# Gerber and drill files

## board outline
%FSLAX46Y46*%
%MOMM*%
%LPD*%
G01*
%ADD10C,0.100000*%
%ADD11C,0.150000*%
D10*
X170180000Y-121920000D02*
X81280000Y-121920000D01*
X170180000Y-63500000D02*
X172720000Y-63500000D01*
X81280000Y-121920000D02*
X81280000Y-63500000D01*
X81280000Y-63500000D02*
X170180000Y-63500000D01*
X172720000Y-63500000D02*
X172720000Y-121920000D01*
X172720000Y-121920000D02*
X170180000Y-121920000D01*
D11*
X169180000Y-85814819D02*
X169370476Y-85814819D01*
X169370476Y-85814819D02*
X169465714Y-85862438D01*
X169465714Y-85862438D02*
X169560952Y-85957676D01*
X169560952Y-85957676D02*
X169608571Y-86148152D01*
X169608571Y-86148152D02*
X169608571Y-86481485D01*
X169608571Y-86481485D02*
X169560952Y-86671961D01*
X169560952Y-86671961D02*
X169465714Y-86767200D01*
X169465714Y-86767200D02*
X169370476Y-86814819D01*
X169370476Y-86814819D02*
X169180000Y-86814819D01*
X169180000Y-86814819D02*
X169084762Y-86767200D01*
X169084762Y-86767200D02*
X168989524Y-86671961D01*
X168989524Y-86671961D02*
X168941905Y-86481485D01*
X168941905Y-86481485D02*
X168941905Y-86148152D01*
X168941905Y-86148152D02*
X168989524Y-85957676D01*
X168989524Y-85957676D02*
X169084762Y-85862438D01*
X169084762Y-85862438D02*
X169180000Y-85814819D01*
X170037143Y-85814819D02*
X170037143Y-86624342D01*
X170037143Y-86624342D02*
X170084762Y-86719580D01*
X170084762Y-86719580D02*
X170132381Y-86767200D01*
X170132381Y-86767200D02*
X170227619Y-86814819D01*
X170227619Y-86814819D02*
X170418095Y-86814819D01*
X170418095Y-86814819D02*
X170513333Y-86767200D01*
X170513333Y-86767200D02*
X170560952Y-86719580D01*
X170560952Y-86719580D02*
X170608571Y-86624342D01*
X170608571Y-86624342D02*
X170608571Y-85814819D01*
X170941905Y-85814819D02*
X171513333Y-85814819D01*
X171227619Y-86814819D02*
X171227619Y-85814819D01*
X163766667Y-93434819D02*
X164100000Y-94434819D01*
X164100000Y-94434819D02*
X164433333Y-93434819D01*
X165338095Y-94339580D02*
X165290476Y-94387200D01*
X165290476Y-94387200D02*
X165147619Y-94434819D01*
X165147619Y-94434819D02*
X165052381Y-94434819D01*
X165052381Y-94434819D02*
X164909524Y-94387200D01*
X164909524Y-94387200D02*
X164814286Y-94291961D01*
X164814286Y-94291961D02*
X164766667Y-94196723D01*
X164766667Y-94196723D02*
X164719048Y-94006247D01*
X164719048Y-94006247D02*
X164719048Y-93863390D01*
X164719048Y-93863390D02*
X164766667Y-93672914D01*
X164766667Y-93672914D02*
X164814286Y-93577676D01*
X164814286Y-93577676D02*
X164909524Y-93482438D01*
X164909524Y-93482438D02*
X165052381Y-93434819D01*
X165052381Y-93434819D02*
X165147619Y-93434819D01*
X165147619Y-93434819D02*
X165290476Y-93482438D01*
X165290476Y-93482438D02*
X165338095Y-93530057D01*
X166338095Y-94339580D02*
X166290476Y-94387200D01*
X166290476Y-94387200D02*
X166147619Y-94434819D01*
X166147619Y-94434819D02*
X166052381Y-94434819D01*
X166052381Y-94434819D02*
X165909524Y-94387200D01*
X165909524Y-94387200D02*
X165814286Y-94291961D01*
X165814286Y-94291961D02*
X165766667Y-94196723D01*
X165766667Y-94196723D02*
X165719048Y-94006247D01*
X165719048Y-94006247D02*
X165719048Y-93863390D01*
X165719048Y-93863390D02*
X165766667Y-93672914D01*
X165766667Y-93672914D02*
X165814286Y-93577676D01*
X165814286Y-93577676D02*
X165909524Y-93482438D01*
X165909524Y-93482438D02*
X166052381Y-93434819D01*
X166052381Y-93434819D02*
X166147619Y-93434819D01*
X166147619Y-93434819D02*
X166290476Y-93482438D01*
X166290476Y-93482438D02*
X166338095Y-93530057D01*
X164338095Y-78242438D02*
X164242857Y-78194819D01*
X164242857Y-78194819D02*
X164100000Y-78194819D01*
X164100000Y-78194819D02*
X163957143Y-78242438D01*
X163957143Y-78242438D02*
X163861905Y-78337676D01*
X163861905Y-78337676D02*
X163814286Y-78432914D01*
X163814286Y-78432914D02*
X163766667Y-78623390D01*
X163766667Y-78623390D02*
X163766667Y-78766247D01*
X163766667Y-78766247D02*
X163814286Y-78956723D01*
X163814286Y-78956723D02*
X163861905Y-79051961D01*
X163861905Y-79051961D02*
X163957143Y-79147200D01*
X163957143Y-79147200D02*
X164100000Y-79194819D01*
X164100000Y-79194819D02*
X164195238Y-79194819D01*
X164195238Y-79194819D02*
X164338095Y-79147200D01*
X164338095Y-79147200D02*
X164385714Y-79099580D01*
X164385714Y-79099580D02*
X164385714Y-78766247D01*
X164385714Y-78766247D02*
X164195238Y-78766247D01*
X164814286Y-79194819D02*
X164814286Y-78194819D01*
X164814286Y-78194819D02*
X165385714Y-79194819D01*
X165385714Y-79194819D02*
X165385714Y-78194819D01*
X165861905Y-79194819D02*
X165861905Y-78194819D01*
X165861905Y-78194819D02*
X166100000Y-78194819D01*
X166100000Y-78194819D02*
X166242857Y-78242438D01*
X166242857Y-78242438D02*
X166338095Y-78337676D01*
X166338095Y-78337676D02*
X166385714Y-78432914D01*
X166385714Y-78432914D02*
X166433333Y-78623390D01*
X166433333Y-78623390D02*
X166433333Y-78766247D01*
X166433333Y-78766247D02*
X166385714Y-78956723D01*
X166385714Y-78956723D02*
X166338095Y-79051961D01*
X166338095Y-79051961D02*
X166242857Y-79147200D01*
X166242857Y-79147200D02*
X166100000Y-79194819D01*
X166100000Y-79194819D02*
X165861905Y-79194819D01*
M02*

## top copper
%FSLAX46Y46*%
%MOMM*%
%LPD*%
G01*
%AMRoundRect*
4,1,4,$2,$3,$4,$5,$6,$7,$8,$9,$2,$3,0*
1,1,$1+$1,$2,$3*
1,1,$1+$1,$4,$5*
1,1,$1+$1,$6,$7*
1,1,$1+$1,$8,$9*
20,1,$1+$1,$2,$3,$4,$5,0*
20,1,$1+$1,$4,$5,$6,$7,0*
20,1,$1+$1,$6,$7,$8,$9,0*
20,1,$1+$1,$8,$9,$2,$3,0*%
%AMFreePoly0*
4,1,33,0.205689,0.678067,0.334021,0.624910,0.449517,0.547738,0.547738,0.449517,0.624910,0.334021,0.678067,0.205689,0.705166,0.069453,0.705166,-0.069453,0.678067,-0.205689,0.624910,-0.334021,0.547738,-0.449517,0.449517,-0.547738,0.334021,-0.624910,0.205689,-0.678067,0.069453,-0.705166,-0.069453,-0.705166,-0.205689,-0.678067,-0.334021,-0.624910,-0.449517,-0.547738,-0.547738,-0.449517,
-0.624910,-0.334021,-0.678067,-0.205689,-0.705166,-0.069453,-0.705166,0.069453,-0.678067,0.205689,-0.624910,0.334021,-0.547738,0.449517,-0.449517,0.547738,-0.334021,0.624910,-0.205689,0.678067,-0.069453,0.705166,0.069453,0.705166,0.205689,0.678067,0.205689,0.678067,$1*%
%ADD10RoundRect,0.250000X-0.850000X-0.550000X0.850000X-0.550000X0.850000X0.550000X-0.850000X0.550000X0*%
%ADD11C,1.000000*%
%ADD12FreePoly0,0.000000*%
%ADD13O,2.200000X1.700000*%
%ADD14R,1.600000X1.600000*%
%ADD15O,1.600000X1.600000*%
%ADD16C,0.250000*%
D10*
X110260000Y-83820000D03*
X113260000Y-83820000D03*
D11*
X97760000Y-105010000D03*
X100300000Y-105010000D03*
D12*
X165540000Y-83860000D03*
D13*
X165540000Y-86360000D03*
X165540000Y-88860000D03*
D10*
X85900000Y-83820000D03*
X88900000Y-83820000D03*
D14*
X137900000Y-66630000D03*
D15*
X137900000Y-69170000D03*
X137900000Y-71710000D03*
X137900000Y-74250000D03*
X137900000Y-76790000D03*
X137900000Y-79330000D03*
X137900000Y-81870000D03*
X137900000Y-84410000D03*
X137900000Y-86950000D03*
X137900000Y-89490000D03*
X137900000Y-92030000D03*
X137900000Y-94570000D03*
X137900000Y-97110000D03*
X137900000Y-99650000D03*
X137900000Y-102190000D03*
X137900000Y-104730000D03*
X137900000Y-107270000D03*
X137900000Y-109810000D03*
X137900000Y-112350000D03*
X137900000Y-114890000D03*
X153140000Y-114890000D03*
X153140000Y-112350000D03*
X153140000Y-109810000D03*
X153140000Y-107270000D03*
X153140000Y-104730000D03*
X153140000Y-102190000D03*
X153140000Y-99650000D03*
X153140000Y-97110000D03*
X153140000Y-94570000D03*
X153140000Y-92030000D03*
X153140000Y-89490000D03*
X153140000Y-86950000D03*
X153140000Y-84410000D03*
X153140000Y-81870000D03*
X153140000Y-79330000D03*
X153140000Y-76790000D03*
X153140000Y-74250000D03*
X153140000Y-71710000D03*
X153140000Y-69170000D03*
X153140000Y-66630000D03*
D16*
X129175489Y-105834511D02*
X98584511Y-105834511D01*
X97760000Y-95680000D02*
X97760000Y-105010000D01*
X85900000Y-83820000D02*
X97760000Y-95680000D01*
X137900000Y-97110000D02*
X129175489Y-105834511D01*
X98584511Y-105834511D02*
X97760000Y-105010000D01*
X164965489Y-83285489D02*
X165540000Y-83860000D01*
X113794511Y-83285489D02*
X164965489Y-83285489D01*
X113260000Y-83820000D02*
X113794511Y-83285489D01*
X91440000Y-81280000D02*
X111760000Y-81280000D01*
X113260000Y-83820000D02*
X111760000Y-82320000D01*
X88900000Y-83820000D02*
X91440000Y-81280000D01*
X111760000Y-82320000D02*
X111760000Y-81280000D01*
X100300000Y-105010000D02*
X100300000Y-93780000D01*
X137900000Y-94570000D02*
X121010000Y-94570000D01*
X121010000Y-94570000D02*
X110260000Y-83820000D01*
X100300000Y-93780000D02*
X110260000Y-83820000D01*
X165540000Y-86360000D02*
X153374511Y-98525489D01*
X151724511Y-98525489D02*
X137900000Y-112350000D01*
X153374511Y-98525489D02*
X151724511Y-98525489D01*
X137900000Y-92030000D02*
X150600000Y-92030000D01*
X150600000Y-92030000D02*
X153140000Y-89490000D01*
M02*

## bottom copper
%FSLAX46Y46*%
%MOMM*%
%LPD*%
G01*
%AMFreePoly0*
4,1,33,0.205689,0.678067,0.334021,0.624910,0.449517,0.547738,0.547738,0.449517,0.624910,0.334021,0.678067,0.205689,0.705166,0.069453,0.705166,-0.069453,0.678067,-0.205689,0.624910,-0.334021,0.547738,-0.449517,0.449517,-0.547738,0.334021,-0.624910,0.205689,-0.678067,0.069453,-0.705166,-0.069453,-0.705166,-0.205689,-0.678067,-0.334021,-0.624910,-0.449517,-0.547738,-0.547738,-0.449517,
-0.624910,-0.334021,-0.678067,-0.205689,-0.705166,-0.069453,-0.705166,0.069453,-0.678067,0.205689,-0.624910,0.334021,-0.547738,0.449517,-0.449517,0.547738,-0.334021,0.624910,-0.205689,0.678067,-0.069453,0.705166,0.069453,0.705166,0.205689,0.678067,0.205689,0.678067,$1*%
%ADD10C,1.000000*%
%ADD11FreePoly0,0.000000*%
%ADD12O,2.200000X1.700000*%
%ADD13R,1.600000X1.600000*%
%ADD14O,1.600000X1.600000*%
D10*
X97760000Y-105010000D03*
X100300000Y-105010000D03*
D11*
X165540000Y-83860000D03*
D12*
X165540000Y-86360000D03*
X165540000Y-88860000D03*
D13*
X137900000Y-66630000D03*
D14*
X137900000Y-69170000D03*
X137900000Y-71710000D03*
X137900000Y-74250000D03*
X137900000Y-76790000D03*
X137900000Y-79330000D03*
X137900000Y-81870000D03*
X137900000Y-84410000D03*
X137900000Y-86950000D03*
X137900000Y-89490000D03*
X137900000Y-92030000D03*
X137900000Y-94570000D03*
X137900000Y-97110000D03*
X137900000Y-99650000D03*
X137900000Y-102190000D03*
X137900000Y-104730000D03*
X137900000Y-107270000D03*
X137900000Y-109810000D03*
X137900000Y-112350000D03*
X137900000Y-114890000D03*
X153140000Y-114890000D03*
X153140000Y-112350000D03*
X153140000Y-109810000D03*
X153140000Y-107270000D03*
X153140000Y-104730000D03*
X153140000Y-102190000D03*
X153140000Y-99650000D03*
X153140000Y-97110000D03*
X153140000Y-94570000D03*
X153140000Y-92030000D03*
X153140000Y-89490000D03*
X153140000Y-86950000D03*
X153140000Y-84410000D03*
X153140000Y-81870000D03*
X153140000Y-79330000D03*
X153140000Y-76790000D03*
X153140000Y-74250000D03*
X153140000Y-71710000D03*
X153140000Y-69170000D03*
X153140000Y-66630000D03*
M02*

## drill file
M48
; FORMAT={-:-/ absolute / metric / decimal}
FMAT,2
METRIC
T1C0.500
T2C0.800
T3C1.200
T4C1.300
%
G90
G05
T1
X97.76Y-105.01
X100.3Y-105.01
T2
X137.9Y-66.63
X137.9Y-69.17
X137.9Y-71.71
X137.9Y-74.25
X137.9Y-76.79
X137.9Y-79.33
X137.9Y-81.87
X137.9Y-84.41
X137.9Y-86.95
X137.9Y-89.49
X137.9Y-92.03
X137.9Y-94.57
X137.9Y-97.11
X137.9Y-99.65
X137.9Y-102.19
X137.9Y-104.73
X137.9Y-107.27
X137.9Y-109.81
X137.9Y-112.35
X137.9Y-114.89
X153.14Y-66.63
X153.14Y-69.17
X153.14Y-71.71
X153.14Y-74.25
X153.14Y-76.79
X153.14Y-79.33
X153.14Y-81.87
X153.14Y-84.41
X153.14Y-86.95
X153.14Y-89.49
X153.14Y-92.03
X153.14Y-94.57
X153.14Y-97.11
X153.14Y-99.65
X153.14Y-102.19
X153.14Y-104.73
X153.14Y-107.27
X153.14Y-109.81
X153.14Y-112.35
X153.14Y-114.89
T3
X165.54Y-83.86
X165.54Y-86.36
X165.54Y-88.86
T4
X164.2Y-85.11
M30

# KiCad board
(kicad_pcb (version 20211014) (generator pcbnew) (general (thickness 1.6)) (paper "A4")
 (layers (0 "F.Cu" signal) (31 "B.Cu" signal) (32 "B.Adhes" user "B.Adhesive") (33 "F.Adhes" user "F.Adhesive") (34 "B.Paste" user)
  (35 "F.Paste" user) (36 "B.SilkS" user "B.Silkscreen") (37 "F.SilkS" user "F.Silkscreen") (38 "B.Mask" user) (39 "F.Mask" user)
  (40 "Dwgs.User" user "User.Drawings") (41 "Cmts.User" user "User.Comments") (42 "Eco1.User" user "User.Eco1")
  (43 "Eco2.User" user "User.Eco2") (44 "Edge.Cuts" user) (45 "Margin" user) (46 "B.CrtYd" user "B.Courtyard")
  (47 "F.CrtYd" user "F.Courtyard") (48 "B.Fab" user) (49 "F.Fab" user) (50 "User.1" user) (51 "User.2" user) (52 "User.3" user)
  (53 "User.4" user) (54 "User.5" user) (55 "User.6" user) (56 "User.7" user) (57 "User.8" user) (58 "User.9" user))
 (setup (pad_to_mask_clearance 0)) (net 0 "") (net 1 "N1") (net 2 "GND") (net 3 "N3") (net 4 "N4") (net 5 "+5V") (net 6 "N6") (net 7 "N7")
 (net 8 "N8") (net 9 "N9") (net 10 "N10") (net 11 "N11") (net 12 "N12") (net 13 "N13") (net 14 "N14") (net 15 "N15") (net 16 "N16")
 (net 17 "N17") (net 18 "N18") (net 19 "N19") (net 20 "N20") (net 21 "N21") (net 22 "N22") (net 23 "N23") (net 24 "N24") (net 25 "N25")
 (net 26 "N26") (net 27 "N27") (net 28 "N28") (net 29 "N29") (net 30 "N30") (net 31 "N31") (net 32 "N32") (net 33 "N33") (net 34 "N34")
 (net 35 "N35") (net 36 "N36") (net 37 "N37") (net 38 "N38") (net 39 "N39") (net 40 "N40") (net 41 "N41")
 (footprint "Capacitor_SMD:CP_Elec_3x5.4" (layer "F.Cu") (at 111.76 83.82)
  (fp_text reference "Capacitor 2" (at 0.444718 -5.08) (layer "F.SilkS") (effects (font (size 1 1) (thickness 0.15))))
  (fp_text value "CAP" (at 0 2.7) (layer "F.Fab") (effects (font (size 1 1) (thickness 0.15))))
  (pad "1" smd roundrect (at -1.5 0) (size 2.2 1.6) (layers "F.Cu" "F.Paste" "F.Mask") (roundrect_rratio 0.15625) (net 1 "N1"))
  (pad "2" smd roundrect (at 1.5 0) (size 2.2 1.6) (layers "F.Cu" "F.Paste" "F.Mask") (roundrect_rratio 0.15625) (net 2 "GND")))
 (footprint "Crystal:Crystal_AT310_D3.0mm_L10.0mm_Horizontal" (layer "F.Cu") (at 97.76 105.01)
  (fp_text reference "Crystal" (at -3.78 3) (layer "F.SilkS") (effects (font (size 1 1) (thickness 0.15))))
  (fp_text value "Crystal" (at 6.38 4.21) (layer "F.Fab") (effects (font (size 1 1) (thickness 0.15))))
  (pad "1" thru_hole circle (at 0 0) (size 1 1) (drill 0.5) (layers *.Cu *.Mask) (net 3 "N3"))
  (pad "2" thru_hole circle (at 2.54 0) (size 1 1) (drill 0.5) (layers *.Cu *.Mask) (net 1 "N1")))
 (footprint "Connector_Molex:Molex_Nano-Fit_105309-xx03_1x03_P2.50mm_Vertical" (layer "F.Cu") (at 165.54 83.86)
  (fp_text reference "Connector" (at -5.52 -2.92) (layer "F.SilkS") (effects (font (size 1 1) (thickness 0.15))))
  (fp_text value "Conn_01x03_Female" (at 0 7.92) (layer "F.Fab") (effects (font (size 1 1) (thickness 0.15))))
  (pad "" np_thru_hole circle (at -1.34 1.25) (size 1.3 1.3) (drill 1.3) (layers *.Cu *.Mask))
  (pad "1" thru_hole custom (at 0 0) (size 1.417157 1.417157) (drill 1.2) (layers *.Cu *.Mask) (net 2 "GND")
   (options (clearance outline) (anchor circle)) (primitives))
  (pad "2" thru_hole oval (at 0 2.5) (size 2.2 1.7) (drill 1.2) (layers *.Cu *.Mask) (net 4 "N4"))
  (pad "3" thru_hole oval (at 0 5) (size 2.2 1.7) (drill 1.2) (layers *.Cu *.Mask) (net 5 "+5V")))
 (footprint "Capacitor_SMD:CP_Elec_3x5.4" (layer "F.Cu") (at 87.4 83.82)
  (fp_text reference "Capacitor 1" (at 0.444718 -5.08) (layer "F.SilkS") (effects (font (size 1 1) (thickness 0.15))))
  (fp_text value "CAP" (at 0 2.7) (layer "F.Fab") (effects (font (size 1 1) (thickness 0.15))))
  (pad "1" smd roundrect (at -1.5 0) (size 2.2 1.6) (layers "F.Cu" "F.Paste" "F.Mask") (roundrect_rratio 0.15625) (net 3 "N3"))
  (pad "2" smd roundrect (at 1.5 0) (size 2.2 1.6) (layers "F.Cu" "F.Paste" "F.Mask") (roundrect_rratio 0.15625) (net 2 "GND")))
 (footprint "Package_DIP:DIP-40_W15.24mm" (layer "F.Cu") (at 137.9 66.63)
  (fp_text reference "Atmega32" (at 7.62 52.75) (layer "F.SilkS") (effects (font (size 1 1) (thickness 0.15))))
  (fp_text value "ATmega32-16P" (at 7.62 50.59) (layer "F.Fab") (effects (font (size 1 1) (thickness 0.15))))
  (pad "1" thru_hole rect (at 0 0) (size 1.6 1.6) (drill 0.8) (layers *.Cu *.Mask) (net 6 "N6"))
  (pad "2" thru_hole oval (at 0 2.54) (size 1.6 1.6) (drill 0.8) (layers *.Cu *.Mask) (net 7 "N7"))
  (pad "3" thru_hole oval (at 0 5.08) (size 1.6 1.6) (drill 0.8) (layers *.Cu *.Mask) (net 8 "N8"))
  (pad "4" thru_hole oval (at 0 7.62) (size 1.6 1.6) (drill 0.8) (layers *.Cu *.Mask) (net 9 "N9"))
  (pad "5" thru_hole oval (at 0 10.16) (size 1.6 1.6) (drill 0.8) (layers *.Cu *.Mask) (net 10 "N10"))
  (pad "6" thru_hole oval (at 0 12.7) (size 1.6 1.6) (drill 0.8) (layers *.Cu *.Mask) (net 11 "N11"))
  (pad "7" thru_hole oval (at 0 15.24) (size 1.6 1.6) (drill 0.8) (layers *.Cu *.Mask) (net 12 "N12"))
  (pad "8" thru_hole oval (at 0 17.78) (size 1.6 1.6) (drill 0.8) (layers *.Cu *.Mask) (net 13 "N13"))
  (pad "9" thru_hole oval (at 0 20.32) (size 1.6 1.6) (drill 0.8) (layers *.Cu *.Mask) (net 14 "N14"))
  (pad "10" thru_hole oval (at 0 22.86) (size 1.6 1.6) (drill 0.8) (layers *.Cu *.Mask) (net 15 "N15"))
  (pad "11" thru_hole oval (at 0 25.4) (size 1.6 1.6) (drill 0.8) (layers *.Cu *.Mask) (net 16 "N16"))
  (pad "12" thru_hole oval (at 0 27.94) (size 1.6 1.6) (drill 0.8) (layers *.Cu *.Mask) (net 1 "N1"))
  (pad "13" thru_hole oval (at 0 30.48) (size 1.6 1.6) (drill 0.8) (layers *.Cu *.Mask) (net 3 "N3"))
  (pad "14" thru_hole oval (at 0 33.02) (size 1.6 1.6) (drill 0.8) (layers *.Cu *.Mask) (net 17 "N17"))
  (pad "15" thru_hole oval (at 0 35.56) (size 1.6 1.6) (drill 0.8) (layers *.Cu *.Mask) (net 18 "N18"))
  (pad "16" thru_hole oval (at 0 38.1) (size 1.6 1.6) (drill 0.8) (layers *.Cu *.Mask) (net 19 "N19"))
  (pad "17" thru_hole oval (at 0 40.64) (size 1.6 1.6) (drill 0.8) (layers *.Cu *.Mask) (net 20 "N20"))
  (pad "18" thru_hole oval (at 0 43.18) (size 1.6 1.6) (drill 0.8) (layers *.Cu *.Mask) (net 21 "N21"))
  (pad "19" thru_hole oval (at 0 45.72) (size 1.6 1.6) (drill 0.8) (layers *.Cu *.Mask) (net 4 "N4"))
  (pad "20" thru_hole oval (at 0 48.26) (size 1.6 1.6) (drill 0.8) (layers *.Cu *.Mask) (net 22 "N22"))
  (pad "21" thru_hole oval (at 15.24 48.26) (size 1.6 1.6) (drill 0.8) (layers *.Cu *.Mask) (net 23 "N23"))
  (pad "22" thru_hole oval (at 15.24 45.72) (size 1.6 1.6) (drill 0.8) (layers *.Cu *.Mask) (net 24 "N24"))
  (pad "23" thru_hole oval (at 15.24 43.18) (size 1.6 1.6) (drill 0.8) (layers *.Cu *.Mask) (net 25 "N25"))
  (pad "24" thru_hole oval (at 15.24 40.64) (size 1.6 1.6) (drill 0.8) (layers *.Cu *.Mask) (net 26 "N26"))
  (pad "25" thru_hole oval (at 15.24 38.1) (size 1.6 1.6) (drill 0.8) (layers *.Cu *.Mask) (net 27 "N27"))
  (pad "26" thru_hole oval (at 15.24 35.56) (size 1.6 1.6) (drill 0.8) (layers *.Cu *.Mask) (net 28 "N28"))
  (pad "27" thru_hole oval (at 15.24 33.02) (size 1.6 1.6) (drill 0.8) (layers *.Cu *.Mask) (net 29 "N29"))
  (pad "28" thru_hole oval (at 15.24 30.48) (size 1.6 1.6) (drill 0.8) (layers *.Cu *.Mask) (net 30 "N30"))
  (pad "29" thru_hole oval (at 15.24 27.94) (size 1.6 1.6) (drill 0.8) (layers *.Cu *.Mask) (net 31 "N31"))
  (pad "30" thru_hole oval (at 15.24 25.4) (size 1.6 1.6) (drill 0.8) (layers *.Cu *.Mask) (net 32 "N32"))
  (pad "31" thru_hole oval (at 15.24 22.86) (size 1.6 1.6) (drill 0.8) (layers *.Cu *.Mask) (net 16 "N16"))
  (pad "32" thru_hole oval (at 15.24 20.32) (size 1.6 1.6) (drill 0.8) (layers *.Cu *.Mask) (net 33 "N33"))
  (pad "33" thru_hole oval (at 15.24 17.78) (size 1.6 1.6) (drill 0.8) (layers *.Cu *.Mask) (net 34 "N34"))
  (pad "34" thru_hole oval (at 15.24 15.24) (size 1.6 1.6) (drill 0.8) (layers *.Cu *.Mask) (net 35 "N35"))
  (pad "35" thru_hole oval (at 15.24 12.7) (size 1.6 1.6) (drill 0.8) (layers *.Cu *.Mask) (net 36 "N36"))
  (pad "36" thru_hole oval (at 15.24 10.16) (size 1.6 1.6) (drill 0.8) (layers *.Cu *.Mask) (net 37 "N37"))
  (pad "37" thru_hole oval (at 15.24 7.62) (size 1.6 1.6) (drill 0.8) (layers *.Cu *.Mask) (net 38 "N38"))
  (pad "38" thru_hole oval (at 15.24 5.08) (size 1.6 1.6) (drill 0.8) (layers *.Cu *.Mask) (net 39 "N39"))
  (pad "39" thru_hole oval (at 15.24 2.54) (size 1.6 1.6) (drill 0.8) (layers *.Cu *.Mask) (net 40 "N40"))
  (pad "40" thru_hole oval (at 15.24 0) (size 1.6 1.6) (drill 0.8) (layers *.Cu *.Mask) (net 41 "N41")))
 (gr_line (start 170.18 121.92) (end 81.28 121.92) (layer "Edge.Cuts") (width 0.1))
 (gr_line (start 170.18 63.5) (end 172.72 63.5) (layer "Edge.Cuts") (width 0.1))
 (gr_line (start 81.28 121.92) (end 81.28 63.5) (layer "Edge.Cuts") (width 0.1))
 (gr_line (start 81.28 63.5) (end 170.18 63.5) (layer "Edge.Cuts") (width 0.1))
 (gr_line (start 172.72 63.5) (end 172.72 121.92) (layer "Edge.Cuts") (width 0.1))
 (gr_line (start 172.72 121.92) (end 170.18 121.92) (layer "Edge.Cuts") (width 0.1))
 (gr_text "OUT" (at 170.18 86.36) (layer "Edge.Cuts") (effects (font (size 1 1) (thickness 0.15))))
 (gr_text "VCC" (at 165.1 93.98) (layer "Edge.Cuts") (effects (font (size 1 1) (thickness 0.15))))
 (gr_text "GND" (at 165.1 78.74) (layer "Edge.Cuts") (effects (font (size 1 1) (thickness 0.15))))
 (segment (start 129.175489 105.834511) (end 98.584511 105.834511) (width 0.25) (layer "F.Cu") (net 3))
 (segment (start 97.76 95.68) (end 97.76 105.01) (width 0.25) (layer "F.Cu") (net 3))
 (segment (start 85.9 83.82) (end 97.76 95.68) (width 0.25) (layer "F.Cu") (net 3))
 (segment (start 137.9 97.11) (end 129.175489 105.834511) (width 0.25) (layer "F.Cu") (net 3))
 (segment (start 98.584511 105.834511) (end 97.76 105.01) (width 0.25) (layer "F.Cu") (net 3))
 (segment (start 164.965489 83.285489) (end 165.54 83.86) (width 0.25) (layer "F.Cu") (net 2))
 (segment (start 113.794511 83.285489) (end 164.965489 83.285489) (width 0.25) (layer "F.Cu") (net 2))
 (segment (start 113.26 83.82) (end 113.794511 83.285489) (width 0.25) (layer "F.Cu") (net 2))
 (segment (start 91.44 81.28) (end 111.76 81.28) (width 0.25) (layer "F.Cu") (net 2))
 (segment (start 113.26 83.82) (end 111.76 82.32) (width 0.25) (layer "F.Cu") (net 2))
 (segment (start 88.9 83.82) (end 91.44 81.28) (width 0.25) (layer "F.Cu") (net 2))
 (segment (start 111.76 82.32) (end 111.76 81.28) (width 0.25) (layer "F.Cu") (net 2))
 (segment (start 100.3 105.01) (end 100.3 93.78) (width 0.25) (layer "F.Cu") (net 1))
 (segment (start 137.9 94.57) (end 121.01 94.57) (width 0.25) (layer "F.Cu") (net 1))
 (segment (start 121.01 94.57) (end 110.26 83.82) (width 0.25) (layer "F.Cu") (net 1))
 (segment (start 100.3 93.78) (end 110.26 83.82) (width 0.25) (layer "F.Cu") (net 1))
 (segment (start 165.54 86.36) (end 153.374511 98.525489) (width 0.25) (layer "F.Cu") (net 4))
 (segment (start 151.724511 98.525489) (end 137.9 112.35) (width 0.25) (layer "F.Cu") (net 4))
 (segment (start 153.374511 98.525489) (end 151.724511 98.525489) (width 0.25) (layer "F.Cu") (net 4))
 (segment (start 137.9 92.03) (end 150.6 92.03) (width 0.25) (layer "F.Cu") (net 16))
 (segment (start 150.6 92.03) (end 153.14 89.49) (width 0.25) (layer "F.Cu") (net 16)))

